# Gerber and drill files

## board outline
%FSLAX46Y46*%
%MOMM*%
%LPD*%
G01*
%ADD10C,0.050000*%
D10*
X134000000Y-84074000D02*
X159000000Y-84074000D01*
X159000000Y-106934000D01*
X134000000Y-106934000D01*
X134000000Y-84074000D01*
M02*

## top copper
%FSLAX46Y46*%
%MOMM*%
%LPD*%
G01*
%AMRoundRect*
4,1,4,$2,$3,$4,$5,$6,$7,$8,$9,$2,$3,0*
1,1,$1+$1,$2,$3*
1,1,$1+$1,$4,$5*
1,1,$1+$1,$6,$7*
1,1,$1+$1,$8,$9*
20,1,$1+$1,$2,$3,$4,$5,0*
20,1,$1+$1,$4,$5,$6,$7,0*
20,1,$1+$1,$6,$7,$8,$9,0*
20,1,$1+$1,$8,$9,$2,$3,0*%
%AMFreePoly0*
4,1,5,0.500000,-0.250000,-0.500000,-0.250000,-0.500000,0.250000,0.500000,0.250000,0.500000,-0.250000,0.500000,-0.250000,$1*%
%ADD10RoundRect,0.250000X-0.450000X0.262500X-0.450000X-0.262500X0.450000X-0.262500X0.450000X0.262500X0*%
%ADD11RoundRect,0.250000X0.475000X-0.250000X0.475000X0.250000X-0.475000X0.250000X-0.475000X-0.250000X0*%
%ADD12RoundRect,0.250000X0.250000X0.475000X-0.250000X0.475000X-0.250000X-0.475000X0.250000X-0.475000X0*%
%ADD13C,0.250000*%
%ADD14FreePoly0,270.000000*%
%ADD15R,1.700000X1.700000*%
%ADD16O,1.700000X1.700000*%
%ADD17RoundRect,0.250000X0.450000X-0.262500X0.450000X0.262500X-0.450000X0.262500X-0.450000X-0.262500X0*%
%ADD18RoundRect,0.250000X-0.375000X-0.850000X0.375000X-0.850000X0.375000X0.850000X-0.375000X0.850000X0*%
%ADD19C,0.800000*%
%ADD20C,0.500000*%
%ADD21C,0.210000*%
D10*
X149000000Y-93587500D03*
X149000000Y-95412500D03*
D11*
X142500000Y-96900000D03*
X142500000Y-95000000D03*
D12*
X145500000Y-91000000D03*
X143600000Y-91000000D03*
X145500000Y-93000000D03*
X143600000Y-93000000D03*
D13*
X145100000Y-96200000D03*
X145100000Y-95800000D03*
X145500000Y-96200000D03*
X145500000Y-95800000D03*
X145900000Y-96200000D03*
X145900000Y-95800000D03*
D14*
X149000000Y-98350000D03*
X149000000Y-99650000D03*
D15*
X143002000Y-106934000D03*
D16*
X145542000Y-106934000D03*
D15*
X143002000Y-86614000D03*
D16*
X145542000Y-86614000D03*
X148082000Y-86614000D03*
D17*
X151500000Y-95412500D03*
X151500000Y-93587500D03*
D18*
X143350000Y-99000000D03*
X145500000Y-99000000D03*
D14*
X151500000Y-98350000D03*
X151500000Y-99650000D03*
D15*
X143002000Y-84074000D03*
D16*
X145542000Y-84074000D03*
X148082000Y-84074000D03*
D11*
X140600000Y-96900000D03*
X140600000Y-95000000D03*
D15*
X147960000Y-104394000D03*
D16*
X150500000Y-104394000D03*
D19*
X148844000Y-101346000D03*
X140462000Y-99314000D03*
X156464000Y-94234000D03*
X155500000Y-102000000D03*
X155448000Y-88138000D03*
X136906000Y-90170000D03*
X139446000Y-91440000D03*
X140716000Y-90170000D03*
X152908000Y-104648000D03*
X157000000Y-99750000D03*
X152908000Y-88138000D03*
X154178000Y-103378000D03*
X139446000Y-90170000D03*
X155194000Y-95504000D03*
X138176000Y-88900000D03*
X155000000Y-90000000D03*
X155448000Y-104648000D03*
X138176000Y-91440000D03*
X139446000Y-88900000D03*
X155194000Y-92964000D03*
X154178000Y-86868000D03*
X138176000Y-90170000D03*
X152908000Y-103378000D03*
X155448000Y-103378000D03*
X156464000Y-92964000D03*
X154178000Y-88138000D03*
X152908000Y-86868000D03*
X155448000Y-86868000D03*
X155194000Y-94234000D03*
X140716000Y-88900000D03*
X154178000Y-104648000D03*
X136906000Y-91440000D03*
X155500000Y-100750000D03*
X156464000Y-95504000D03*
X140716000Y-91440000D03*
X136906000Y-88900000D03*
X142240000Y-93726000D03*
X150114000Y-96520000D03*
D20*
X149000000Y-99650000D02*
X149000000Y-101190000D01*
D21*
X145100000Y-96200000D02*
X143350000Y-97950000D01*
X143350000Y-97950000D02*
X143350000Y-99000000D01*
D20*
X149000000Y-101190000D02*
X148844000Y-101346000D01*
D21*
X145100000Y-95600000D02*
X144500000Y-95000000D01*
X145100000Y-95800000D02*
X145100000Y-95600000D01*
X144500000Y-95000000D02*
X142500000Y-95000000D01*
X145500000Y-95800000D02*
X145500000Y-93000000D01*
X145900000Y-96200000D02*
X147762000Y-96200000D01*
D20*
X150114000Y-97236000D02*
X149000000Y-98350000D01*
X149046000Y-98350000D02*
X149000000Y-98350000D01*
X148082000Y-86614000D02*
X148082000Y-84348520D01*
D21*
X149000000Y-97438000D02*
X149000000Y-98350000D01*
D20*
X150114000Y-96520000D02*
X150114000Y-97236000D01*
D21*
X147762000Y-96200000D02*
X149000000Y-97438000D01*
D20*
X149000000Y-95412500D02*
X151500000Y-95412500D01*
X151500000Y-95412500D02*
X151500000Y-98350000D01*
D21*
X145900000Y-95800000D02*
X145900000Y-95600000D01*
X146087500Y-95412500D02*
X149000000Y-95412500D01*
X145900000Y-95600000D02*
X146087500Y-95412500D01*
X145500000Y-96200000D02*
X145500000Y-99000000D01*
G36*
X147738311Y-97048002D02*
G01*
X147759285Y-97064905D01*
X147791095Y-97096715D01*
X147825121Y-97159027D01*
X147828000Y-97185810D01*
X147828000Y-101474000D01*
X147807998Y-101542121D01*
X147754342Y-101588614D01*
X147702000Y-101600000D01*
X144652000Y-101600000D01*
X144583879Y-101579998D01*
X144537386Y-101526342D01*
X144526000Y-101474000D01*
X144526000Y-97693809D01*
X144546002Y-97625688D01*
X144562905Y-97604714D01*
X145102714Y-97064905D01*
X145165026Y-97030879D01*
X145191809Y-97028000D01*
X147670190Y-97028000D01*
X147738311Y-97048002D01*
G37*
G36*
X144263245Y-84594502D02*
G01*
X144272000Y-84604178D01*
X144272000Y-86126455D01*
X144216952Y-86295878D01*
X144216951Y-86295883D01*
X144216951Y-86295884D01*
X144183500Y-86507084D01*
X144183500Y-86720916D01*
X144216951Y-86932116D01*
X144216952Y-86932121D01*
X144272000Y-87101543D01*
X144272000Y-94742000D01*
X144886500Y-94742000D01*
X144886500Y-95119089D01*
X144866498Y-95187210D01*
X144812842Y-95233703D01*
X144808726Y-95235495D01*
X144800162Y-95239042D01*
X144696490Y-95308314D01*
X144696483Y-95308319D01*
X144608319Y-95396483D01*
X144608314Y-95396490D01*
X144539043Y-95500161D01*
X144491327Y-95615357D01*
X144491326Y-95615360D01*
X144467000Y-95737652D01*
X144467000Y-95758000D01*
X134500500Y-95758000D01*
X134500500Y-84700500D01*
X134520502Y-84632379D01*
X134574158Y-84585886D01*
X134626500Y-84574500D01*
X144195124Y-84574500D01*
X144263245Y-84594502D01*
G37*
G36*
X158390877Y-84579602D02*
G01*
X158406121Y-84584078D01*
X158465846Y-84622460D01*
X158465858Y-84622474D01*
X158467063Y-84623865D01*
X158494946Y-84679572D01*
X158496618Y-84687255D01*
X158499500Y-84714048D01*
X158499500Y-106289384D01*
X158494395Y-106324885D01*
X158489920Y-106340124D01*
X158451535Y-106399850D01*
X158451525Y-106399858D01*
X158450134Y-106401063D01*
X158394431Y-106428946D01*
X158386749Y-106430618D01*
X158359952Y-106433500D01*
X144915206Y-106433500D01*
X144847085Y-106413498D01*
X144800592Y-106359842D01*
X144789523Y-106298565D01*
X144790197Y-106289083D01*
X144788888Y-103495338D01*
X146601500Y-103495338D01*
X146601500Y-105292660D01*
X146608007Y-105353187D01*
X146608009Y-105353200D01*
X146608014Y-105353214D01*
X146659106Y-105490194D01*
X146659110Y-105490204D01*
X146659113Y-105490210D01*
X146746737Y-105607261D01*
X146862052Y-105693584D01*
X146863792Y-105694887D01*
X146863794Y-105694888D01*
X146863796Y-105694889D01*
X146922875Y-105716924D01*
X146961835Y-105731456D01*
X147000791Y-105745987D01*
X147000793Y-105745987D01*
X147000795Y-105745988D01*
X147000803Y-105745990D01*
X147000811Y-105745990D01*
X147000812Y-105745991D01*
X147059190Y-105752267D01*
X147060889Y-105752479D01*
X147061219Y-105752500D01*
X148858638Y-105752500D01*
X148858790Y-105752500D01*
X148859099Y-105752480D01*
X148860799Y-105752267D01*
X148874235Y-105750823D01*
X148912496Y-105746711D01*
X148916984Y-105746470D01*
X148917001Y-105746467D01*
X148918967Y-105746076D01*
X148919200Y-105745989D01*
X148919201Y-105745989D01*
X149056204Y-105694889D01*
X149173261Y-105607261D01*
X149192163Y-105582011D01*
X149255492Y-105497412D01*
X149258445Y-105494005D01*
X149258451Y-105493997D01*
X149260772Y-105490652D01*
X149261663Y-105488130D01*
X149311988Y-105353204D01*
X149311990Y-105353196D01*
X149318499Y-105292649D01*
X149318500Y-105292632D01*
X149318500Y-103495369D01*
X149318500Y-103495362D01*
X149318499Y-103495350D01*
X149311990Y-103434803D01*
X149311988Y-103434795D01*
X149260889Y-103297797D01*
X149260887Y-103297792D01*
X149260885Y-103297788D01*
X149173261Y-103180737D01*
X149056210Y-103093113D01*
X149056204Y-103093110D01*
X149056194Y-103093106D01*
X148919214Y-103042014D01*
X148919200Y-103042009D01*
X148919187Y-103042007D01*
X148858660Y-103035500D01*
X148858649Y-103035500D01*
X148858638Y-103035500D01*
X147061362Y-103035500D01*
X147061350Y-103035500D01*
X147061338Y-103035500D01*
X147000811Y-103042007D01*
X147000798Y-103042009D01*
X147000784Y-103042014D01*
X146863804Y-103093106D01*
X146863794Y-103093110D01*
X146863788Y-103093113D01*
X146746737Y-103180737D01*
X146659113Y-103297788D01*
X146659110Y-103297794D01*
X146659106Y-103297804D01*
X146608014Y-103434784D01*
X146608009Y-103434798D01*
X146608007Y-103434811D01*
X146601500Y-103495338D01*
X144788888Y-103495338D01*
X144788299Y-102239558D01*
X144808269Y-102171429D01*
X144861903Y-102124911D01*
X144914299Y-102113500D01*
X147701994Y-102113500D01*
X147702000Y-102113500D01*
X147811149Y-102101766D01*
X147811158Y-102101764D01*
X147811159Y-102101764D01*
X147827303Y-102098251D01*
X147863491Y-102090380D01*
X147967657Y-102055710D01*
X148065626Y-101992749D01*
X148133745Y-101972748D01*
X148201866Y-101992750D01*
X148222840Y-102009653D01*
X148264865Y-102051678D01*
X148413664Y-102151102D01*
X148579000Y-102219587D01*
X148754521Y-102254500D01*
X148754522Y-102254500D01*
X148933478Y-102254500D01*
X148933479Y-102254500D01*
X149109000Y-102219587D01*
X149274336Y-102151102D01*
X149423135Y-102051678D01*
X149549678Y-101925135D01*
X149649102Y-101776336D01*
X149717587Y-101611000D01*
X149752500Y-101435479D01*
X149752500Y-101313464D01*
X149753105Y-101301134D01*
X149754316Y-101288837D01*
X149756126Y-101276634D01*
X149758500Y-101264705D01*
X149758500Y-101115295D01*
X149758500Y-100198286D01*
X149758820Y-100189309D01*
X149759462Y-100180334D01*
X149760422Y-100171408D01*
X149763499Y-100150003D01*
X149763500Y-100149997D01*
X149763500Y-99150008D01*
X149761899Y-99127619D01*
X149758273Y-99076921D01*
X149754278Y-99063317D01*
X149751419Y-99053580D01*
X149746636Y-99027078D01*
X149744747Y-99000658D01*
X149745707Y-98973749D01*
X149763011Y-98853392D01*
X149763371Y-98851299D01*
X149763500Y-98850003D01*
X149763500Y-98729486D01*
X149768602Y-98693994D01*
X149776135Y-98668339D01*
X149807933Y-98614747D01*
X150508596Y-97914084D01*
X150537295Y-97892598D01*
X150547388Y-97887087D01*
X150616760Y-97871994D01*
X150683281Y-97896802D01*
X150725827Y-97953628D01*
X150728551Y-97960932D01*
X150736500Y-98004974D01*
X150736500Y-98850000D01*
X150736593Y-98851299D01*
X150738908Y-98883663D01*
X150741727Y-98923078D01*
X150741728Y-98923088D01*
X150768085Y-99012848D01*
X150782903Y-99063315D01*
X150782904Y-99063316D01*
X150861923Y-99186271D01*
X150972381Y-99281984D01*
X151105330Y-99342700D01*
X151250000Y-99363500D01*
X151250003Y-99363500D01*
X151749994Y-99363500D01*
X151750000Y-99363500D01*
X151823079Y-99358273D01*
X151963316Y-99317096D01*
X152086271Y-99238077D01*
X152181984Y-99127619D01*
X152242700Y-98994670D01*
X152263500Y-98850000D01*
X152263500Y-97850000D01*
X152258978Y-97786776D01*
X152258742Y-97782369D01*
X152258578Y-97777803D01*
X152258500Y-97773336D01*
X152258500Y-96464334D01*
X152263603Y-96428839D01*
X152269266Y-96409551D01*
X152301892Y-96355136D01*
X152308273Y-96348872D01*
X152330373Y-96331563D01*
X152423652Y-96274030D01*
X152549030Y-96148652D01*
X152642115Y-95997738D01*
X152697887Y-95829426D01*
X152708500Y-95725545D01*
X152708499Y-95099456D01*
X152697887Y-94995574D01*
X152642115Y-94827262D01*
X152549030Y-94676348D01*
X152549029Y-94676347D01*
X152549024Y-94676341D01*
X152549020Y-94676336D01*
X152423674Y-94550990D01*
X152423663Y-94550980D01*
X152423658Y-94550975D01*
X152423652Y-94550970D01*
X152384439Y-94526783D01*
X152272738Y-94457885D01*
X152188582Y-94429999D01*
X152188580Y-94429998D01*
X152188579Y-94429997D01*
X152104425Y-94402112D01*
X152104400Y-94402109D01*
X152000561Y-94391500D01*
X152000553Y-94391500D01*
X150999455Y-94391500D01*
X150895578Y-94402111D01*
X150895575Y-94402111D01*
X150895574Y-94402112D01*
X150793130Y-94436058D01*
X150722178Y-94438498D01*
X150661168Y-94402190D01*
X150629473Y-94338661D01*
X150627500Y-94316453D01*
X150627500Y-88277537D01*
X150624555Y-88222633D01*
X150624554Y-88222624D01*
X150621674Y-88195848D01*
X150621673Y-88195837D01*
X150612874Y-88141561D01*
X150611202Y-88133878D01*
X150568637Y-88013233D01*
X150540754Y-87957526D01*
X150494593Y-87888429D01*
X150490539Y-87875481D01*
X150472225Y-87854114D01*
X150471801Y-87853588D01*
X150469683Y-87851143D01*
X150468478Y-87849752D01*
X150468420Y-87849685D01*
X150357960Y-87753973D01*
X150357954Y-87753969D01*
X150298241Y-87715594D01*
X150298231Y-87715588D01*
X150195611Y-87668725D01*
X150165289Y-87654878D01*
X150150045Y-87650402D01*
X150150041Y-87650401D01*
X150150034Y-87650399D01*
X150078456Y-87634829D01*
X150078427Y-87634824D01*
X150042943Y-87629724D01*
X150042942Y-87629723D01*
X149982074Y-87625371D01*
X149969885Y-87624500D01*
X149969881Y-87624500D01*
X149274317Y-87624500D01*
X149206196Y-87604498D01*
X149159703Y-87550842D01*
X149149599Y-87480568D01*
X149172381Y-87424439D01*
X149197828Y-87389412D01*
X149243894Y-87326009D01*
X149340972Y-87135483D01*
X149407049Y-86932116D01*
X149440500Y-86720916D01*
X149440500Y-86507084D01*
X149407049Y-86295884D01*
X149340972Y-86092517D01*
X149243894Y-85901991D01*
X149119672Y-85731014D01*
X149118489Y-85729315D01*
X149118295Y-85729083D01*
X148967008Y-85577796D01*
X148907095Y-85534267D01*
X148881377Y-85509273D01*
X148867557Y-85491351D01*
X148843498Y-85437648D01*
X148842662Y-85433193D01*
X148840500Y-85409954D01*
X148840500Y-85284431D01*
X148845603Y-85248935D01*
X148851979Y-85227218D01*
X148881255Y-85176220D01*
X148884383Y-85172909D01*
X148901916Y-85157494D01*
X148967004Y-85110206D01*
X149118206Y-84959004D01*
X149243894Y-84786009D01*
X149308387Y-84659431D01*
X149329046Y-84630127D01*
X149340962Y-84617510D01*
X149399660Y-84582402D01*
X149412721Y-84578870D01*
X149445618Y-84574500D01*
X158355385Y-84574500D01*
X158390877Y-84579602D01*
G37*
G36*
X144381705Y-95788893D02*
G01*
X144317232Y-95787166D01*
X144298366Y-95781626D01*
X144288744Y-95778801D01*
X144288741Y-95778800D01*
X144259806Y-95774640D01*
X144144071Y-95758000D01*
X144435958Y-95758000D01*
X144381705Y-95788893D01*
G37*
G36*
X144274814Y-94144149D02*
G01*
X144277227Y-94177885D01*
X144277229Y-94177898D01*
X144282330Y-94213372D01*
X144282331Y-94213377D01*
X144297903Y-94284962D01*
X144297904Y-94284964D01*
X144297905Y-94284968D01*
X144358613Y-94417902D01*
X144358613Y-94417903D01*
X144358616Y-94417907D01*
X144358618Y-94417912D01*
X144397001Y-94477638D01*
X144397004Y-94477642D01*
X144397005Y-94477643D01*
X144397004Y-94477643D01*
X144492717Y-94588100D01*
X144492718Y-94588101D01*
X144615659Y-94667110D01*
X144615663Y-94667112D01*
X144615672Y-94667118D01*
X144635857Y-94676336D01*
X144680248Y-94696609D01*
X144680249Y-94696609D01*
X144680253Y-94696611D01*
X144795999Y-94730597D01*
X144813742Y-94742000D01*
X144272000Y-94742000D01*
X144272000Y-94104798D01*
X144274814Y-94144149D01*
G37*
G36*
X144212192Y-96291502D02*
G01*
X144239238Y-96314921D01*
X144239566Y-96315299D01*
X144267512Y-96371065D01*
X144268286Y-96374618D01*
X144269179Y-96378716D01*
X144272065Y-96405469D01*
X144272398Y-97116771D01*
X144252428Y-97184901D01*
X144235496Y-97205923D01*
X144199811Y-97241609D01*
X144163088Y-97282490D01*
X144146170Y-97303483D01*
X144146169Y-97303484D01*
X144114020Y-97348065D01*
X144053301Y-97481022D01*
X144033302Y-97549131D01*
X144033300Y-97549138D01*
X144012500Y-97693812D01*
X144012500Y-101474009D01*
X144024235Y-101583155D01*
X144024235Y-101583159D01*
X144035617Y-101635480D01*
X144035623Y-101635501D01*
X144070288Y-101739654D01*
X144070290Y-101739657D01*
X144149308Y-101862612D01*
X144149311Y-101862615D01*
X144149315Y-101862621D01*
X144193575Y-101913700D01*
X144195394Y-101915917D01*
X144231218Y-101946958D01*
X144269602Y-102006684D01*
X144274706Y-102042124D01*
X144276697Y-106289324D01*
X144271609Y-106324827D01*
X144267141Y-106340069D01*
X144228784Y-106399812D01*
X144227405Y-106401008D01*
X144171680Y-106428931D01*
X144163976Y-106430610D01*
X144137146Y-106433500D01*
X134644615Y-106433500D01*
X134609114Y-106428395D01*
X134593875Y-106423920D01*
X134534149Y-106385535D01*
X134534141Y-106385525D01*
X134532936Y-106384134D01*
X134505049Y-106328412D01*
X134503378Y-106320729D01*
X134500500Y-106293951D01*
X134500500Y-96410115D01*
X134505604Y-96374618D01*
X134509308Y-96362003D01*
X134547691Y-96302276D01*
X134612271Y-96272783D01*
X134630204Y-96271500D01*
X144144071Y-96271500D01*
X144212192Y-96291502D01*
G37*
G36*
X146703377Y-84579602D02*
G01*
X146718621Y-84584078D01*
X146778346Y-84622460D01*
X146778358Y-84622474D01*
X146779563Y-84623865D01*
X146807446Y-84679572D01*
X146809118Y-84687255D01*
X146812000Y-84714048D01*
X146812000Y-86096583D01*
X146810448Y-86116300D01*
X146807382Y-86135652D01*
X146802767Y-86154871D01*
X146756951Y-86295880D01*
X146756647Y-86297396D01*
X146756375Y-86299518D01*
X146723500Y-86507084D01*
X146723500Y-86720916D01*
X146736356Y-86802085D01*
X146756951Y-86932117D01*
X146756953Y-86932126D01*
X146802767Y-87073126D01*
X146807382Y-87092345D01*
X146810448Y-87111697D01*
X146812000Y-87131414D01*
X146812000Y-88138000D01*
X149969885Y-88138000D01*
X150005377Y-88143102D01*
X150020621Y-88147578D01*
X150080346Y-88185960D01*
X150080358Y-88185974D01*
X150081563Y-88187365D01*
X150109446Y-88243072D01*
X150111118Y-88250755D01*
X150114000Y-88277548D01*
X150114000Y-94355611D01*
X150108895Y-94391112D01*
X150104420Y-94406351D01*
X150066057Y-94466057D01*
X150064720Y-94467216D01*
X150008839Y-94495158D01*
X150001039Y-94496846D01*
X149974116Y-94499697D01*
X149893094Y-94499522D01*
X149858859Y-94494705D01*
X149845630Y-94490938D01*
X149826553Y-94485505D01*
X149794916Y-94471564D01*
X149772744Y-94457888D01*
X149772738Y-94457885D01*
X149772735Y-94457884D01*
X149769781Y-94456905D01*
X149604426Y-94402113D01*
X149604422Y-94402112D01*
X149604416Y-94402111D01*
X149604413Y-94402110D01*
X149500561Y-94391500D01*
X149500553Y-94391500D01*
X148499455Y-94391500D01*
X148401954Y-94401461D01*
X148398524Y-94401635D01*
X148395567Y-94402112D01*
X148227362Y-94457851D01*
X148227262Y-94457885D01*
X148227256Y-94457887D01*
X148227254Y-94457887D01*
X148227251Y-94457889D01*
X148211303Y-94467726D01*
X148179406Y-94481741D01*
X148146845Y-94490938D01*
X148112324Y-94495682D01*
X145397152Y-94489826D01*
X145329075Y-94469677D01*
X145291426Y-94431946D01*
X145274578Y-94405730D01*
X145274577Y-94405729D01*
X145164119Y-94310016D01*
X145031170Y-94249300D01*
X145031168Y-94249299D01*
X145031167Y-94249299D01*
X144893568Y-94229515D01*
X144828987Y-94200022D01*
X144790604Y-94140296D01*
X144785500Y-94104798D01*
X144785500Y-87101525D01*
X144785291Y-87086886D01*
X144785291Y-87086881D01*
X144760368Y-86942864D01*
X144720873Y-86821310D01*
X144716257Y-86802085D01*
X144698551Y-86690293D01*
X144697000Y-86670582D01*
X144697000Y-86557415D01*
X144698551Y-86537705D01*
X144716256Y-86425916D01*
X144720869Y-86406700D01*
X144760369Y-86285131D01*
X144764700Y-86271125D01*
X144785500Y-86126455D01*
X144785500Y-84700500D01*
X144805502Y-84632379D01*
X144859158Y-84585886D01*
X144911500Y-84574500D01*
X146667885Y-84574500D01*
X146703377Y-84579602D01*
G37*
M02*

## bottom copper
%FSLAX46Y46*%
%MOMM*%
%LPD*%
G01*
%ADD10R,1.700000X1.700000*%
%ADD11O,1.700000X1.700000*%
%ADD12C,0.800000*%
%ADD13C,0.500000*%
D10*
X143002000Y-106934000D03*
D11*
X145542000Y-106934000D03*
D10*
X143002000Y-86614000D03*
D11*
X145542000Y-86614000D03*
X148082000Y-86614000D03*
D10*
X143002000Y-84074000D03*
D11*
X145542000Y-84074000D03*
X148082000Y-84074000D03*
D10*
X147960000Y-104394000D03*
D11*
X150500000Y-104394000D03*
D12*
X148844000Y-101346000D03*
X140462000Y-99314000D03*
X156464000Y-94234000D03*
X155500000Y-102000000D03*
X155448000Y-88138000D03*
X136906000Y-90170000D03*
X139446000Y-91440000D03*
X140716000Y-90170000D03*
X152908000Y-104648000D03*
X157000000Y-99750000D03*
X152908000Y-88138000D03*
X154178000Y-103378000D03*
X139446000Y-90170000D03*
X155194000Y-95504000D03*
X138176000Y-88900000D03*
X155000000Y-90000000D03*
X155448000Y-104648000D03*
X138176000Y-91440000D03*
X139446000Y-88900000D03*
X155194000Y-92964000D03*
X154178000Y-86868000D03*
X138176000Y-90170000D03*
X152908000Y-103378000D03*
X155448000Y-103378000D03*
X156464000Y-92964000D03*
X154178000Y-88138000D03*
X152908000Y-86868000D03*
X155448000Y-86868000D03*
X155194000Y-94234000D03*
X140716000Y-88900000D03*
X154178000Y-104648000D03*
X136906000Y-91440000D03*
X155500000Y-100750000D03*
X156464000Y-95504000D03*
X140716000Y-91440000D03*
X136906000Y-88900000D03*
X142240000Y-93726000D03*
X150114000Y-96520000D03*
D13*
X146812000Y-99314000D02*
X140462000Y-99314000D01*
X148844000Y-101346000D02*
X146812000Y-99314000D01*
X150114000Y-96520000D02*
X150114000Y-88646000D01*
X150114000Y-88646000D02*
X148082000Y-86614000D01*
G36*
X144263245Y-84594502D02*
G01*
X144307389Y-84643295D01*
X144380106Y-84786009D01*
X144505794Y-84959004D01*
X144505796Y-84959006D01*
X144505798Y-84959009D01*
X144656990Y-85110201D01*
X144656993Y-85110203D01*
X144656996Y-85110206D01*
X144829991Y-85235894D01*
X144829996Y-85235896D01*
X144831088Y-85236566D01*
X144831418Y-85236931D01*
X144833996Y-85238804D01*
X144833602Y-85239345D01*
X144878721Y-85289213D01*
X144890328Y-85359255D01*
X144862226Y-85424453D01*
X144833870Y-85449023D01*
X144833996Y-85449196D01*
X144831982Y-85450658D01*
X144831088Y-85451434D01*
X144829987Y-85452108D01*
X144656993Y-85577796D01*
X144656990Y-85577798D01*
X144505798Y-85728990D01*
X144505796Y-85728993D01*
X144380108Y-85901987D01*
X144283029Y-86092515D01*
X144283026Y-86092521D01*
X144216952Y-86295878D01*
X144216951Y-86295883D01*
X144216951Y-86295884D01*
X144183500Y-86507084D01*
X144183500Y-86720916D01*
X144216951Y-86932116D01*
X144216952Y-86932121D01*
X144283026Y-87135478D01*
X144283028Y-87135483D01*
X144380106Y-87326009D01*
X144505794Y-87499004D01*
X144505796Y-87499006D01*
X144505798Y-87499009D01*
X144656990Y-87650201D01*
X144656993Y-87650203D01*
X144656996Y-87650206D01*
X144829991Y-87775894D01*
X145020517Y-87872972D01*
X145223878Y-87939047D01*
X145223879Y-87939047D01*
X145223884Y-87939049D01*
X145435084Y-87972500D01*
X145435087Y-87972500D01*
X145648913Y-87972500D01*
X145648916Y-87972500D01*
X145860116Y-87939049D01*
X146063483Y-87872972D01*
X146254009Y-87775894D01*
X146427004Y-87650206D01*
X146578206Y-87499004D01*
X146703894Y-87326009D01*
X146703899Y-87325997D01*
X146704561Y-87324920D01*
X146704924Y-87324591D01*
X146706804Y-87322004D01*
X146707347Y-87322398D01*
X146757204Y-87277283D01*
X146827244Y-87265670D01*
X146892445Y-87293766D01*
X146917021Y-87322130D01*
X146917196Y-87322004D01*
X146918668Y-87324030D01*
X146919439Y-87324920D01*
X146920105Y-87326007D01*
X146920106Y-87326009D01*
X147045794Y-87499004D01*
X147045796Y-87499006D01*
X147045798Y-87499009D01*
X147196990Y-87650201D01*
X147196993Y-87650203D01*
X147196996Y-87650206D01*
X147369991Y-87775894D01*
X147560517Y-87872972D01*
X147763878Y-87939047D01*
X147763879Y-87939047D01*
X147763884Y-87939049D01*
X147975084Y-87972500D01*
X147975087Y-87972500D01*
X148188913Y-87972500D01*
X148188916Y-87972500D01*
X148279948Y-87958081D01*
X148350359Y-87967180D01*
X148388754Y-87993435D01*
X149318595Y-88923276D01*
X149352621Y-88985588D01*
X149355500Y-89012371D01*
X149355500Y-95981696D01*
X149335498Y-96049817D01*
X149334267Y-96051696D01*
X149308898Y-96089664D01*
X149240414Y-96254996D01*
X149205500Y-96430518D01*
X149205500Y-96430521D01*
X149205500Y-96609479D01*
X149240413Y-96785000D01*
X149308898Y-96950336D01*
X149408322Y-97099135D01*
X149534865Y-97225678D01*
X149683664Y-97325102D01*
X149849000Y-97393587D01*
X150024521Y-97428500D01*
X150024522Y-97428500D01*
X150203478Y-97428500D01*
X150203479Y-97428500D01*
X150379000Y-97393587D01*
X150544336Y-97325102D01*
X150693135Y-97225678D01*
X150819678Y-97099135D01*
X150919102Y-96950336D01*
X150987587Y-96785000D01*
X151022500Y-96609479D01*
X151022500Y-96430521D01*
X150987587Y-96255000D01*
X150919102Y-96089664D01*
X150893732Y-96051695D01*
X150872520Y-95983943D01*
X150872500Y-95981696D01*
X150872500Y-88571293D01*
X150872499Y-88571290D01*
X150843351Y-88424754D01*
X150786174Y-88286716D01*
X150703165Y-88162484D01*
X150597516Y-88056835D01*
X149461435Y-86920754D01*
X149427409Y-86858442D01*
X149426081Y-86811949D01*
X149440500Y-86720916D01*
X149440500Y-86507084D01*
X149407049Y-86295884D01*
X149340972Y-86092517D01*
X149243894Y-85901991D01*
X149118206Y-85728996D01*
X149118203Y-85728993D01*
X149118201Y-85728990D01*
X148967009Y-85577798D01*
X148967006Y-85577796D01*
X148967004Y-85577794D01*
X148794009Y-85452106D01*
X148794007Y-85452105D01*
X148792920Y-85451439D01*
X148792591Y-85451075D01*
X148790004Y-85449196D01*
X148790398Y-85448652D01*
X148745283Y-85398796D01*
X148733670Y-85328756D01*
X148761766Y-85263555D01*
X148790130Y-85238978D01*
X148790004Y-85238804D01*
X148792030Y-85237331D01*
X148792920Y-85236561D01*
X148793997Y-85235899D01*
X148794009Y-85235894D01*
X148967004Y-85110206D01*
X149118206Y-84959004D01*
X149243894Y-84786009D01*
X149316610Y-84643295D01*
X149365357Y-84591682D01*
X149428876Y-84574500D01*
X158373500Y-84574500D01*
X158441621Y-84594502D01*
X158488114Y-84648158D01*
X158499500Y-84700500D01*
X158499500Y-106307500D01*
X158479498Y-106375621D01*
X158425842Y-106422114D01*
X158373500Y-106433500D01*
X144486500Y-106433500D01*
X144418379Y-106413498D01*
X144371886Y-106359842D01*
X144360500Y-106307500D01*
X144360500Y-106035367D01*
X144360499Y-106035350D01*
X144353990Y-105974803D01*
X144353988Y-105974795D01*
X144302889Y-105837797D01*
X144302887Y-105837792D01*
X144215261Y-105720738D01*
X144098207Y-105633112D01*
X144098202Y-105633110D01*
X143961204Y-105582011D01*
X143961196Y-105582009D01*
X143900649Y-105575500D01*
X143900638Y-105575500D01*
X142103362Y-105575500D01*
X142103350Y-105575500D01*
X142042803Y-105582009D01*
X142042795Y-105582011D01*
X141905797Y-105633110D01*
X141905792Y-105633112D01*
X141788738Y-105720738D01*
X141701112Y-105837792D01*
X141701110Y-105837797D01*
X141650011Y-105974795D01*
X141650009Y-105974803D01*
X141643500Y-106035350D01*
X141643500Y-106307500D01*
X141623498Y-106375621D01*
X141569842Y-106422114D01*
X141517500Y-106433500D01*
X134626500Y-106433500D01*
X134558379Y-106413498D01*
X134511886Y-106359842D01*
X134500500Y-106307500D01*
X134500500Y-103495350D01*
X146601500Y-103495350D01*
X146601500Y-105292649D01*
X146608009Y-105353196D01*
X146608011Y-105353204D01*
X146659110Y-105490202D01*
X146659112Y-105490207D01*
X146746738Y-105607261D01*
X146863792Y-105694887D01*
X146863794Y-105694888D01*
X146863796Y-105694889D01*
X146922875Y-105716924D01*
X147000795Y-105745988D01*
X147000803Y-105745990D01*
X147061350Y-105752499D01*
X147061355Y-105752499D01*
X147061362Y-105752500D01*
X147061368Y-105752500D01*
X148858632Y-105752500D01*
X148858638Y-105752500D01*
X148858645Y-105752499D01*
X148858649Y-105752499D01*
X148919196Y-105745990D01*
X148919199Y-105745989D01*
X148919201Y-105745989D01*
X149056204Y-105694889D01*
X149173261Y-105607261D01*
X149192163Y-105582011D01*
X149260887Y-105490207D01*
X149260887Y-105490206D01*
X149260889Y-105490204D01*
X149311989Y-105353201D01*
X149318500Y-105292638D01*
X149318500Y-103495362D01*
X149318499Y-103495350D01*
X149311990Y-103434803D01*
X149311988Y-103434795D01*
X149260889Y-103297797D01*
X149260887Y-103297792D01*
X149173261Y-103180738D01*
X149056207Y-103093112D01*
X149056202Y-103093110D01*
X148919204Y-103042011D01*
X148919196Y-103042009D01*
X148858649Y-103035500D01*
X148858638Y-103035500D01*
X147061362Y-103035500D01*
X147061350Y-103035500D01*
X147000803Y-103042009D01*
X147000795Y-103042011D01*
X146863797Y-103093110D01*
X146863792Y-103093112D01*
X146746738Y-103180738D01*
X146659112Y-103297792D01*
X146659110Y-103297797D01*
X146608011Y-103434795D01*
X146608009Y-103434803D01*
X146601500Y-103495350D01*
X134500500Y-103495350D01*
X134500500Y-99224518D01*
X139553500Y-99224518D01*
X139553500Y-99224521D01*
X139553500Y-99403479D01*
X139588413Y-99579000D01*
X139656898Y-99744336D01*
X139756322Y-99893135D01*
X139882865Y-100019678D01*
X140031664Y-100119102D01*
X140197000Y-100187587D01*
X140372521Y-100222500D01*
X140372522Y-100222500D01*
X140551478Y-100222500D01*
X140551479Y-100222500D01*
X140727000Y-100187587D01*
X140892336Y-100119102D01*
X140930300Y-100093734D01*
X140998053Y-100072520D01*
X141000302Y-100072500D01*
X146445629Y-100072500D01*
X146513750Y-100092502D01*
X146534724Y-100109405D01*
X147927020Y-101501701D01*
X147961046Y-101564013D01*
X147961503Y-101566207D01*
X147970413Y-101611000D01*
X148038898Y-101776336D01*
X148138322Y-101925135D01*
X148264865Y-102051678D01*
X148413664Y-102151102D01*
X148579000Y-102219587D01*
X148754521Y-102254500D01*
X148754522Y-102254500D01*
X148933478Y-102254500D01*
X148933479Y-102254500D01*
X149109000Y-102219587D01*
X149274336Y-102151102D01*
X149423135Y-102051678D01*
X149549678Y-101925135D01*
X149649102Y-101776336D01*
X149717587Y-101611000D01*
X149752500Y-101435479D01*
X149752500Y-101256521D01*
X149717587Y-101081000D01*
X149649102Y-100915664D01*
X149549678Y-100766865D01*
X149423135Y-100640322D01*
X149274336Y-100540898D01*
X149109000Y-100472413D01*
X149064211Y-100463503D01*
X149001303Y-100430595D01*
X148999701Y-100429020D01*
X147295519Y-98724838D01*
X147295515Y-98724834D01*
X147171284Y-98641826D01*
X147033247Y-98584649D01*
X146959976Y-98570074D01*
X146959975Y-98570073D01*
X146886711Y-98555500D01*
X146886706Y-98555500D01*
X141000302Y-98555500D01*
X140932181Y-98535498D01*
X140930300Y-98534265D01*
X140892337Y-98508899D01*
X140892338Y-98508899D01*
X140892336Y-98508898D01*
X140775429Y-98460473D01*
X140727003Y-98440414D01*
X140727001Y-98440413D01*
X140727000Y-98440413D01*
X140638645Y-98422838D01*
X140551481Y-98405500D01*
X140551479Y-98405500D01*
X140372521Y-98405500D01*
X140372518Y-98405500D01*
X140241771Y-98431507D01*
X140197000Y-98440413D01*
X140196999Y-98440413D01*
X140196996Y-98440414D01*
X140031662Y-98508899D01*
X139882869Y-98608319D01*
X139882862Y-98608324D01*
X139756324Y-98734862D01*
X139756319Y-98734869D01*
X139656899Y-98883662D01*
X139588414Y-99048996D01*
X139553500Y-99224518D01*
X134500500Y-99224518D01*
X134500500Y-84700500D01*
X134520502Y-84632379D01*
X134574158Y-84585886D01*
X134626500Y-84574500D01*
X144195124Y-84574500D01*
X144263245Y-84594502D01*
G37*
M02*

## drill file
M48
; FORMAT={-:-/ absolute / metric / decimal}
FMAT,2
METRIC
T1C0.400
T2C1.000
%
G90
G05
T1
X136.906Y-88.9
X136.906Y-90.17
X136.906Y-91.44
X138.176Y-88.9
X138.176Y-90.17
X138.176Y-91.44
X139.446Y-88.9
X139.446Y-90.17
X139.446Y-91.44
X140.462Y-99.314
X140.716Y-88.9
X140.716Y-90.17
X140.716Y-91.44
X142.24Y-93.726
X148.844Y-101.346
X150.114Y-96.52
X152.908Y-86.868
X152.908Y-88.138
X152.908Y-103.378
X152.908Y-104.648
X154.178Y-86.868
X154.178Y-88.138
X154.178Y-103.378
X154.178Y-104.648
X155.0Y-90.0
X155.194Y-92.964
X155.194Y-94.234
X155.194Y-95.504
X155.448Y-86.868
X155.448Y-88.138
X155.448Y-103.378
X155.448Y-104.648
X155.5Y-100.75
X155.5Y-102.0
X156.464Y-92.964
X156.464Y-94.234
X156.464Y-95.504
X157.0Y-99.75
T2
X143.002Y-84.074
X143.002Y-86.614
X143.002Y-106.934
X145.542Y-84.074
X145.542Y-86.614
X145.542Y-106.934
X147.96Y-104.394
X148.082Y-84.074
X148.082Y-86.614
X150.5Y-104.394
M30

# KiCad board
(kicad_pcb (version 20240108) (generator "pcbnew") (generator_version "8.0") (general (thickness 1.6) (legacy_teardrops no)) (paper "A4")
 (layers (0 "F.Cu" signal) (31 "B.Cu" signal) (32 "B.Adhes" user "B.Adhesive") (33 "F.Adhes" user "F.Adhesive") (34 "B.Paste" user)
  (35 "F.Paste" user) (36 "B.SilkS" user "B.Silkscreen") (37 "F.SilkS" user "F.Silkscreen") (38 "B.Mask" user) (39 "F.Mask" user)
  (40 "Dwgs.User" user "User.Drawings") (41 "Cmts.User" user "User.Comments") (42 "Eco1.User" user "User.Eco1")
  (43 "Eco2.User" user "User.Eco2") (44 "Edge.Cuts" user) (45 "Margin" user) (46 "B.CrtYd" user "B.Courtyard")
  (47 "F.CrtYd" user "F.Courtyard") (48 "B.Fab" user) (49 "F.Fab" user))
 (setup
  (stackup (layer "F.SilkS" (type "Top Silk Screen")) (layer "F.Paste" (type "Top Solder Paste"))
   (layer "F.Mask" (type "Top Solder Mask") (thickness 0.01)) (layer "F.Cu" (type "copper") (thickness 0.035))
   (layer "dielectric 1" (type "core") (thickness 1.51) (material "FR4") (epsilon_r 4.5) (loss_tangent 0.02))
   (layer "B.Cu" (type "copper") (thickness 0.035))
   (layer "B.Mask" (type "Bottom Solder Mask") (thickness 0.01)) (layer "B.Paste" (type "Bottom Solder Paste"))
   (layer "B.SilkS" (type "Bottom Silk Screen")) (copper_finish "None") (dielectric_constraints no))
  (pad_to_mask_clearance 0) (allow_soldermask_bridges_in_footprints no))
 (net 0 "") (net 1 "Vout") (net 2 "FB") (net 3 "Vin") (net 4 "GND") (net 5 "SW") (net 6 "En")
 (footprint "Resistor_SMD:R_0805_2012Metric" (layer "F.Cu") (at 149 94.5 -90)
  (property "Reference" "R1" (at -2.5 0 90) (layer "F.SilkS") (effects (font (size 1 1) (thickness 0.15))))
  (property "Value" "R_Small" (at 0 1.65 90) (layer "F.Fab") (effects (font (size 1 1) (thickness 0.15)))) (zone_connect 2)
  (pad "1" smd roundrect (at -0.9125 0 270) (size 1.025 1.4) (layers "F.Cu" "F.Paste" "F.Mask") (roundrect_rratio 0.243902) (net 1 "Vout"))
  (pad "2" smd roundrect (at 0.9125 0 270) (size 1.025 1.4) (layers "F.Cu" "F.Paste" "F.Mask") (roundrect_rratio 0.243902) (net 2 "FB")))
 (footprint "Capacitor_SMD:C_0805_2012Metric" (layer "F.Cu") (at 142.5 95.95 90)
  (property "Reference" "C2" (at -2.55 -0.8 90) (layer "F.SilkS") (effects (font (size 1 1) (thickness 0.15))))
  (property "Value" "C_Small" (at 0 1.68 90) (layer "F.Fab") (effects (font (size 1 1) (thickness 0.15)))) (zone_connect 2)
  (pad "1" smd roundrect (at -0.95 0 90) (size 1 1.45) (layers "F.Cu" "F.Paste" "F.Mask") (roundrect_rratio 0.25) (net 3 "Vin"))
  (pad "2" smd roundrect (at 0.95 0 90) (size 1 1.45) (layers "F.Cu" "F.Paste" "F.Mask") (roundrect_rratio 0.25) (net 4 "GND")))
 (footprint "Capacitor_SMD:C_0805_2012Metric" (layer "F.Cu") (at 144.55 91 180)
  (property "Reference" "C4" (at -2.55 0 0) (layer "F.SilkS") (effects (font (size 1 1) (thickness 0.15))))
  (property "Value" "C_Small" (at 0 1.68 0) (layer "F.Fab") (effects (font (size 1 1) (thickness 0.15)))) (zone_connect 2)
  (pad "1" smd roundrect (at -0.95 0 180) (size 1 1.45) (layers "F.Cu" "F.Paste" "F.Mask") (roundrect_rratio 0.25) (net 1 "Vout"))
  (pad "2" smd roundrect (at 0.95 0 180) (size 1 1.45) (layers "F.Cu" "F.Paste" "F.Mask") (roundrect_rratio 0.25) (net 4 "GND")))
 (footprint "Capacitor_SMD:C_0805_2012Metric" (layer "F.Cu") (at 144.55 93 180)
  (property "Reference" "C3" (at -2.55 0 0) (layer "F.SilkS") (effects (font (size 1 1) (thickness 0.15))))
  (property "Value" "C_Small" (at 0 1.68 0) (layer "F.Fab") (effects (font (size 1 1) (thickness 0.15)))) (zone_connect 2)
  (pad "1" smd roundrect (at -0.95 0 180) (size 1 1.45) (layers "F.Cu" "F.Paste" "F.Mask") (roundrect_rratio 0.25) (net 1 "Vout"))
  (pad "2" smd roundrect (at 0.95 0 180) (size 1 1.45) (layers "F.Cu" "F.Paste" "F.Mask") (roundrect_rratio 0.25) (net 4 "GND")))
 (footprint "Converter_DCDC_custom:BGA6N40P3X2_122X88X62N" (layer "F.Cu") (at 145.5 96 90)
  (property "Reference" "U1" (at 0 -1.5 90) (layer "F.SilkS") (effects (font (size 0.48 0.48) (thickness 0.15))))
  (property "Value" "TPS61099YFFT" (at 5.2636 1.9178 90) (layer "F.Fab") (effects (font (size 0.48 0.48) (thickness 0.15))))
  (pad "A1" smd circle (at -0.2 -0.4 90) (size 0.25 0.25) (layers "F.Cu" "F.Paste" "F.Mask") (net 3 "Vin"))
  (pad "A2" smd circle (at 0.2 -0.4 90) (size 0.25 0.25) (layers "F.Cu" "F.Paste" "F.Mask") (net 4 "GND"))
  (pad "B1" smd circle (at -0.2 0 90) (size 0.25 0.25) (layers "F.Cu" "F.Paste" "F.Mask") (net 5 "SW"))
  (pad "B2" smd circle (at 0.2 0 90) (size 0.25 0.25) (layers "F.Cu" "F.Paste" "F.Mask") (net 1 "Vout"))
  (pad "C1" smd circle (at -0.2 0.4 90) (size 0.25 0.25) (layers "F.Cu" "F.Paste" "F.Mask") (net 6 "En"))
  (pad "C2" smd circle (at 0.2 0.4 90) (size 0.25 0.25) (layers "F.Cu" "F.Paste" "F.Mask") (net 2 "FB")))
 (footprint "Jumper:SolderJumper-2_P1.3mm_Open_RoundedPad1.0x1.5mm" (layer "F.Cu") (at 149 99 -90)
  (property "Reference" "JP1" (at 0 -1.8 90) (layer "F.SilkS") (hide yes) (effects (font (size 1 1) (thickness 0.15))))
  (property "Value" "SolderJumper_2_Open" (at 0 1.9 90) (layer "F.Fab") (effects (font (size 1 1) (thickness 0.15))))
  (pad "1" smd custom (at -0.65 0 270) (size 1 0.5) (layers "F.Cu" "F.Mask") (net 6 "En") (zone_connect 2)
   (options (clearance outline) (anchor rect)) (primitives))
  (pad "2" smd custom (at 0.65 0 270) (size 1 0.5) (layers "F.Cu" "F.Mask") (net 3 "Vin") (zone_connect 2)
   (options (clearance outline) (anchor rect)) (primitives)))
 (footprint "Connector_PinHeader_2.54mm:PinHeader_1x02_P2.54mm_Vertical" (layer "F.Cu") (at 143.002 106.934 90)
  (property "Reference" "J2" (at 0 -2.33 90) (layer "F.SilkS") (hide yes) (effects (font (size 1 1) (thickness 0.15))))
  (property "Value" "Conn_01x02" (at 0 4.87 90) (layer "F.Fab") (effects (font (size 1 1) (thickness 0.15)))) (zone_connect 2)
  (pad "1" thru_hole rect (at 0 0 90) (size 1.7 1.7) (drill 1) (layers "*.Cu" "*.Mask") (remove_unused_layers no) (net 3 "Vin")
   (zone_connect 2))
  (pad "2" thru_hole oval (at 0 2.54 90) (size 1.7 1.7) (drill 1) (layers "*.Cu" "*.Mask") (remove_unused_layers no) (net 4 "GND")
   (zone_connect 2)))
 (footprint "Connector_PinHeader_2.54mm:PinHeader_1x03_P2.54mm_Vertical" (layer "F.Cu") (at 143.002 86.614 90)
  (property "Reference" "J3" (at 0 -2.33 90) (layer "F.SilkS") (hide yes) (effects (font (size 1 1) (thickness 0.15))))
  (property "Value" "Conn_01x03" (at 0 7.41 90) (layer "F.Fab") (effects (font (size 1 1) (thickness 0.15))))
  (pad "1" thru_hole rect (at 0 0 90) (size 1.7 1.7) (drill 1) (layers "*.Cu" "*.Mask") (remove_unused_layers no) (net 4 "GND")
   (zone_connect 2))
  (pad "2" thru_hole oval (at 0 2.54 90) (size 1.7 1.7) (drill 1) (layers "*.Cu" "*.Mask") (remove_unused_layers no) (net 1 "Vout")
   (zone_connect 2))
  (pad "3" thru_hole oval (at 0 5.08 90) (size 1.7 1.7) (drill 1) (layers "*.Cu" "*.Mask") (remove_unused_layers no) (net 6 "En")))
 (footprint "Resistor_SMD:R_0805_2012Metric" (layer "F.Cu") (at 151.5 94.5 90)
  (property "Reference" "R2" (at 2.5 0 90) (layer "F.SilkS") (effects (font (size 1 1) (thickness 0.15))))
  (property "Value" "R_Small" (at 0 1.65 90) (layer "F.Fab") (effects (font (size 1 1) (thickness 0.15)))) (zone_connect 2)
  (pad "1" smd roundrect (at -0.9125 0 90) (size 1.025 1.4) (layers "F.Cu" "F.Paste" "F.Mask") (roundrect_rratio 0.243902) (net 2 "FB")
   (zone_connect 2))
  (pad "2" smd roundrect (at 0.9125 0 90) (size 1.025 1.4) (layers "F.Cu" "F.Paste" "F.Mask") (roundrect_rratio 0.243902) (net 4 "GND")
   (zone_connect 2)))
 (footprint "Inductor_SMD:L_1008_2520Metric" (layer "F.Cu") (at 144.425 99)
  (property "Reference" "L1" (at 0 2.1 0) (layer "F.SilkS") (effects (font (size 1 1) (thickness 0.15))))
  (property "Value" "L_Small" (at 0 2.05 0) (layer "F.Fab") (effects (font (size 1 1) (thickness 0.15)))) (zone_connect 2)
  (pad "1" smd roundrect (at -1.075 0) (size 1.25 2.2) (layers "F.Cu" "F.Paste" "F.Mask") (roundrect_rratio 0.2) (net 3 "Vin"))
  (pad "2" smd roundrect (at 1.075 0) (size 1.25 2.2) (layers "F.Cu" "F.Paste" "F.Mask") (roundrect_rratio 0.2) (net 5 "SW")))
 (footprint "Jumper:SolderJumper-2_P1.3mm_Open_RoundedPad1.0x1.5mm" (layer "F.Cu") (at 151.5 99 -90)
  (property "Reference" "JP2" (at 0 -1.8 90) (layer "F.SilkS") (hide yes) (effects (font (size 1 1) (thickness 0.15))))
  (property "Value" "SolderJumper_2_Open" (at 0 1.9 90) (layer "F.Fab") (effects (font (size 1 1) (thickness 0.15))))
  (pad "1" smd custom (at -0.65 0 270) (size 1 0.5) (layers "F.Cu" "F.Mask") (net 2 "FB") (zone_connect 2)
   (options (clearance outline) (anchor rect)) (primitives))
  (pad "2" smd custom (at 0.65 0 270) (size 1 0.5) (layers "F.Cu" "F.Mask") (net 4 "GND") (zone_connect 2)
   (options (clearance outline) (anchor rect)) (primitives)))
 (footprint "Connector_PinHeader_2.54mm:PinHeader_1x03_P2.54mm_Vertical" (layer "F.Cu") (at 143.002 84.074 90)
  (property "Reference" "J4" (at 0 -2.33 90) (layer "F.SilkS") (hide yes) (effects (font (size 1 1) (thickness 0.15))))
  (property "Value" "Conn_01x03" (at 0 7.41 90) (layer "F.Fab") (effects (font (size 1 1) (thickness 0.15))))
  (pad "1" thru_hole rect (at 0 0 90) (size 1.7 1.7) (drill 1) (layers "*.Cu" "*.Mask") (remove_unused_layers no) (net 4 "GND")
   (zone_connect 2))
  (pad "2" thru_hole oval (at 0 2.54 90) (size 1.7 1.7) (drill 1) (layers "*.Cu" "*.Mask") (remove_unused_layers no) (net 1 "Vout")
   (zone_connect 2))
  (pad "3" thru_hole oval (at 0 5.08 90) (size 1.7 1.7) (drill 1) (layers "*.Cu" "*.Mask") (remove_unused_layers no) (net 6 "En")))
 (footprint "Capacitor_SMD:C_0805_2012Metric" (layer "F.Cu") (at 140.6 95.95 90)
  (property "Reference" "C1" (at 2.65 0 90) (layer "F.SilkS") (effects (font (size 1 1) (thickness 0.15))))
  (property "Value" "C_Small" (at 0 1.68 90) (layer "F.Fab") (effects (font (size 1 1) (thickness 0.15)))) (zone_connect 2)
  (pad "1" smd roundrect (at -0.95 0 90) (size 1 1.45) (layers "F.Cu" "F.Paste" "F.Mask") (roundrect_rratio 0.25) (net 3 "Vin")
   (zone_connect 2))
  (pad "2" smd roundrect (at 0.95 0 90) (size 1 1.45) (layers "F.Cu" "F.Paste" "F.Mask") (roundrect_rratio 0.25) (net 4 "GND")
   (zone_connect 2)))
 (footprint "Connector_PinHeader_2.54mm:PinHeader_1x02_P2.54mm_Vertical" (layer "F.Cu") (at 147.96 104.394 90)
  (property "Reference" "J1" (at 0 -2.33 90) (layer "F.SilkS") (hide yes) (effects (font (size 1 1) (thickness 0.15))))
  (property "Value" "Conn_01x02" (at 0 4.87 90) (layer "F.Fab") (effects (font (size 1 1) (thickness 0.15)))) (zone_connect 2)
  (pad "1" thru_hole rect (at 0 0 90) (size 1.7 1.7) (drill 1) (layers "*.Cu" "*.Mask") (remove_unused_layers no) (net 3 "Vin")
   (zone_connect 2))
  (pad "2" thru_hole oval (at 0 2.54 90) (size 1.7 1.7) (drill 1) (layers "*.Cu" "*.Mask") (remove_unused_layers no) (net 4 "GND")
   (zone_connect 2)))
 (gr_rect (start 134 84.074) (end 159 106.934) (stroke (width 0.05) (type solid)) (fill none) (layer "Edge.Cuts"))
 (segment (start 149 99.65) (end 149 101.19) (width 0.5) (layer "F.Cu") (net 3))
 (segment (start 145.1 96.2) (end 143.35 97.95) (width 0.21) (layer "F.Cu") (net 3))
 (segment (start 143.35 97.95) (end 143.35 99) (width 0.21) (layer "F.Cu") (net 3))
 (segment (start 149 101.19) (end 148.844 101.346) (width 0.5) (layer "F.Cu") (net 3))
 (via (at 148.844 101.346) (size 0.8) (drill 0.4) (layers "F.Cu" "B.Cu") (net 3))
 (via (at 140.462 99.314) (size 0.8) (drill 0.4) (layers "F.Cu" "B.Cu") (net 3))
 (segment (start 146.812 99.314) (end 140.462 99.314) (width 0.5) (layer "B.Cu") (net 3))
 (segment (start 148.844 101.346) (end 146.812 99.314) (width 0.5) (layer "B.Cu") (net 3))
 (segment (start 145.1 95.6) (end 144.5 95) (width 0.21) (layer "F.Cu") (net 4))
 (segment (start 145.1 95.8) (end 145.1 95.6) (width 0.21) (layer "F.Cu") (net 4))
 (segment (start 144.5 95) (end 142.5 95) (width 0.21) (layer "F.Cu") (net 4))
 (via (at 156.464 94.234) (size 0.8) (drill 0.4) (layers "F.Cu" "B.Cu") (free yes) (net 4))
 (via (at 155.5 102) (size 0.8) (drill 0.4) (layers "F.Cu" "B.Cu") (free yes) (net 4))
 (via (at 155.448 88.138) (size 0.8) (drill 0.4) (layers "F.Cu" "B.Cu") (free yes) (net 4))
 (via (at 136.906 90.17) (size 0.8) (drill 0.4) (layers "F.Cu" "B.Cu") (free yes) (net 4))
 (via (at 139.446 91.44) (size 0.8) (drill 0.4) (layers "F.Cu" "B.Cu") (free yes) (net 4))
 (via (at 140.716 90.17) (size 0.8) (drill 0.4) (layers "F.Cu" "B.Cu") (free yes) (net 4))
 (via (at 152.908 104.648) (size 0.8) (drill 0.4) (layers "F.Cu" "B.Cu") (free yes) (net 4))
 (via (at 157 99.75) (size 0.8) (drill 0.4) (layers "F.Cu" "B.Cu") (free yes) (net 4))
 (via (at 152.908 88.138) (size 0.8) (drill 0.4) (layers "F.Cu" "B.Cu") (free yes) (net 4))
 (via (at 154.178 103.378) (size 0.8) (drill 0.4) (layers "F.Cu" "B.Cu") (free yes) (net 4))
 (via (at 139.446 90.17) (size 0.8) (drill 0.4) (layers "F.Cu" "B.Cu") (free yes) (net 4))
 (via (at 155.194 95.504) (size 0.8) (drill 0.4) (layers "F.Cu" "B.Cu") (free yes) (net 4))
 (via (at 138.176 88.9) (size 0.8) (drill 0.4) (layers "F.Cu" "B.Cu") (free yes) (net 4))
 (via (at 155 90) (size 0.8) (drill 0.4) (layers "F.Cu" "B.Cu") (free yes) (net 4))
 (via (at 155.448 104.648) (size 0.8) (drill 0.4) (layers "F.Cu" "B.Cu") (free yes) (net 4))
 (via (at 138.176 91.44) (size 0.8) (drill 0.4) (layers "F.Cu" "B.Cu") (free yes) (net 4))
 (via (at 139.446 88.9) (size 0.8) (drill 0.4) (layers "F.Cu" "B.Cu") (free yes) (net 4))
 (via (at 155.194 92.964) (size 0.8) (drill 0.4) (layers "F.Cu" "B.Cu") (free yes) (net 4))
 (via (at 154.178 86.868) (size 0.8) (drill 0.4) (layers "F.Cu" "B.Cu") (free yes) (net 4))
 (via (at 138.176 90.17) (size 0.8) (drill 0.4) (layers "F.Cu" "B.Cu") (free yes) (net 4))
 (via (at 152.908 103.378) (size 0.8) (drill 0.4) (layers "F.Cu" "B.Cu") (free yes) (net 4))
 (via (at 155.448 103.378) (size 0.8) (drill 0.4) (layers "F.Cu" "B.Cu") (free yes) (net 4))
 (via (at 156.464 92.964) (size 0.8) (drill 0.4) (layers "F.Cu" "B.Cu") (free yes) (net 4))
 (via (at 154.178 88.138) (size 0.8) (drill 0.4) (layers "F.Cu" "B.Cu") (free yes) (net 4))
 (via (at 152.908 86.868) (size 0.8) (drill 0.4) (layers "F.Cu" "B.Cu") (free yes) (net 4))
 (via (at 155.448 86.868) (size 0.8) (drill 0.4) (layers "F.Cu" "B.Cu") (free yes) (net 4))
 (via (at 155.194 94.234) (size 0.8) (drill 0.4) (layers "F.Cu" "B.Cu") (free yes) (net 4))
 (via (at 140.716 88.9) (size 0.8) (drill 0.4) (layers "F.Cu" "B.Cu") (free yes) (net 4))
 (via (at 154.178 104.648) (size 0.8) (drill 0.4) (layers "F.Cu" "B.Cu") (free yes) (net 4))
 (via (at 136.906 91.44) (size 0.8) (drill 0.4) (layers "F.Cu" "B.Cu") (free yes) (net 4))
 (via (at 155.5 100.75) (size 0.8) (drill 0.4) (layers "F.Cu" "B.Cu") (free yes) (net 4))
 (via (at 156.464 95.504) (size 0.8) (drill 0.4) (layers "F.Cu" "B.Cu") (free yes) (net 4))
 (via (at 140.716 91.44) (size 0.8) (drill 0.4) (layers "F.Cu" "B.Cu") (free yes) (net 4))
 (via (at 136.906 88.9) (size 0.8) (drill 0.4) (layers "F.Cu" "B.Cu") (free yes) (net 4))
 (via (at 142.24 93.726) (size 0.8) (drill 0.4) (layers "F.Cu" "B.Cu") (free yes) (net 4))
 (segment (start 145.5 95.8) (end 145.5 93) (width 0.21) (layer "F.Cu") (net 1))
 (segment (start 145.9 96.2) (end 147.762 96.2) (width 0.21) (layer "F.Cu") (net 6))
 (segment (start 150.114 97.236) (end 149 98.35) (width 0.5) (layer "F.Cu") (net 6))
 (segment (start 149.046 98.35) (end 149 98.35) (width 0.5) (layer "F.Cu") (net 6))
 (segment (start 148.082 86.614) (end 148.082 84.34852) (width 0.5) (layer "F.Cu") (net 6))
 (segment (start 149 97.438) (end 149 98.35) (width 0.21) (layer "F.Cu") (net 6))
 (segment (start 150.114 96.52) (end 150.114 97.236) (width 0.5) (layer "F.Cu") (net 6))
 (segment (start 147.762 96.2) (end 149 97.438) (width 0.21) (layer "F.Cu") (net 6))
 (via (at 150.114 96.52) (size 0.8) (drill 0.4) (layers "F.Cu" "B.Cu") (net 6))
 (segment (start 150.114 96.52) (end 150.114 88.646) (width 0.5) (layer "B.Cu") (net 6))
 (segment (start 150.114 88.646) (end 148.082 86.614) (width 0.5) (layer "B.Cu") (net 6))
 (segment (start 149 95.4125) (end 151.5 95.4125) (width 0.5) (layer "F.Cu") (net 2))
 (segment (start 151.5 95.4125) (end 151.5 98.35) (width 0.5) (layer "F.Cu") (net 2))
 (segment (start 145.9 95.8) (end 145.9 95.6) (width 0.21) (layer "F.Cu") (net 2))
 (segment (start 146.0875 95.4125) (end 149 95.4125) (width 0.21) (layer "F.Cu") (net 2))
 (segment (start 145.9 95.6) (end 146.0875 95.4125) (width 0.21) (layer "F.Cu") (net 2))
 (segment (start 145.5 96.2) (end 145.5 99) (width 0.21) (layer "F.Cu") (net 5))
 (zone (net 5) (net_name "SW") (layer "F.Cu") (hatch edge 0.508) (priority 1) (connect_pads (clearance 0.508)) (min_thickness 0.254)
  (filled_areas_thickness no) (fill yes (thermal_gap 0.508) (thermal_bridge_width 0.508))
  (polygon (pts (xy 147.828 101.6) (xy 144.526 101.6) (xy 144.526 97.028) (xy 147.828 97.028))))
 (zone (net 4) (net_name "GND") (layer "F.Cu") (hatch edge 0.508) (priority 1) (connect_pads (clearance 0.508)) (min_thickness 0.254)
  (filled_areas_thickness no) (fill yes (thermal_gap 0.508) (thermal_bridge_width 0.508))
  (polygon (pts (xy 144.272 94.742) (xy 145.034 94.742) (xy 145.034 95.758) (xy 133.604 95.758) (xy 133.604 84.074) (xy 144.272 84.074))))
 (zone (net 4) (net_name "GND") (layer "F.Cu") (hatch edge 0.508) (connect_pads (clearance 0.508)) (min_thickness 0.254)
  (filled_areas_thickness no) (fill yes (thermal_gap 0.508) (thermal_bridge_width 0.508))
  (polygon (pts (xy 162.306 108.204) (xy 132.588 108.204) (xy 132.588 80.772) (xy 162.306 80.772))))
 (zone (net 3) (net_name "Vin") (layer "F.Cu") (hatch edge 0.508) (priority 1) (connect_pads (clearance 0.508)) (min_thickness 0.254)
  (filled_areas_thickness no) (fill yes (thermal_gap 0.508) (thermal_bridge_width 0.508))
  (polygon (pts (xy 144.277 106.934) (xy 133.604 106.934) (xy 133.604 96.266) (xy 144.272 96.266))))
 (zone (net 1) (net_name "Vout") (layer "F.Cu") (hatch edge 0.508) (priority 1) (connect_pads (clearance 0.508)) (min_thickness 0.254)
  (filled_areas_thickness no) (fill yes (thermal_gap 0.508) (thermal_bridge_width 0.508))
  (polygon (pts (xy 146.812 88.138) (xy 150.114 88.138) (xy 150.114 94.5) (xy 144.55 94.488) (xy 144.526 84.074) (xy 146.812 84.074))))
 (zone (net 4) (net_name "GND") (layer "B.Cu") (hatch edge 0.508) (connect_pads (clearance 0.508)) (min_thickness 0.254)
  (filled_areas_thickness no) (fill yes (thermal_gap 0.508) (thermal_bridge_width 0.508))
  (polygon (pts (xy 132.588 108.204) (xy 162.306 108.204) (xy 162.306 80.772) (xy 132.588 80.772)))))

